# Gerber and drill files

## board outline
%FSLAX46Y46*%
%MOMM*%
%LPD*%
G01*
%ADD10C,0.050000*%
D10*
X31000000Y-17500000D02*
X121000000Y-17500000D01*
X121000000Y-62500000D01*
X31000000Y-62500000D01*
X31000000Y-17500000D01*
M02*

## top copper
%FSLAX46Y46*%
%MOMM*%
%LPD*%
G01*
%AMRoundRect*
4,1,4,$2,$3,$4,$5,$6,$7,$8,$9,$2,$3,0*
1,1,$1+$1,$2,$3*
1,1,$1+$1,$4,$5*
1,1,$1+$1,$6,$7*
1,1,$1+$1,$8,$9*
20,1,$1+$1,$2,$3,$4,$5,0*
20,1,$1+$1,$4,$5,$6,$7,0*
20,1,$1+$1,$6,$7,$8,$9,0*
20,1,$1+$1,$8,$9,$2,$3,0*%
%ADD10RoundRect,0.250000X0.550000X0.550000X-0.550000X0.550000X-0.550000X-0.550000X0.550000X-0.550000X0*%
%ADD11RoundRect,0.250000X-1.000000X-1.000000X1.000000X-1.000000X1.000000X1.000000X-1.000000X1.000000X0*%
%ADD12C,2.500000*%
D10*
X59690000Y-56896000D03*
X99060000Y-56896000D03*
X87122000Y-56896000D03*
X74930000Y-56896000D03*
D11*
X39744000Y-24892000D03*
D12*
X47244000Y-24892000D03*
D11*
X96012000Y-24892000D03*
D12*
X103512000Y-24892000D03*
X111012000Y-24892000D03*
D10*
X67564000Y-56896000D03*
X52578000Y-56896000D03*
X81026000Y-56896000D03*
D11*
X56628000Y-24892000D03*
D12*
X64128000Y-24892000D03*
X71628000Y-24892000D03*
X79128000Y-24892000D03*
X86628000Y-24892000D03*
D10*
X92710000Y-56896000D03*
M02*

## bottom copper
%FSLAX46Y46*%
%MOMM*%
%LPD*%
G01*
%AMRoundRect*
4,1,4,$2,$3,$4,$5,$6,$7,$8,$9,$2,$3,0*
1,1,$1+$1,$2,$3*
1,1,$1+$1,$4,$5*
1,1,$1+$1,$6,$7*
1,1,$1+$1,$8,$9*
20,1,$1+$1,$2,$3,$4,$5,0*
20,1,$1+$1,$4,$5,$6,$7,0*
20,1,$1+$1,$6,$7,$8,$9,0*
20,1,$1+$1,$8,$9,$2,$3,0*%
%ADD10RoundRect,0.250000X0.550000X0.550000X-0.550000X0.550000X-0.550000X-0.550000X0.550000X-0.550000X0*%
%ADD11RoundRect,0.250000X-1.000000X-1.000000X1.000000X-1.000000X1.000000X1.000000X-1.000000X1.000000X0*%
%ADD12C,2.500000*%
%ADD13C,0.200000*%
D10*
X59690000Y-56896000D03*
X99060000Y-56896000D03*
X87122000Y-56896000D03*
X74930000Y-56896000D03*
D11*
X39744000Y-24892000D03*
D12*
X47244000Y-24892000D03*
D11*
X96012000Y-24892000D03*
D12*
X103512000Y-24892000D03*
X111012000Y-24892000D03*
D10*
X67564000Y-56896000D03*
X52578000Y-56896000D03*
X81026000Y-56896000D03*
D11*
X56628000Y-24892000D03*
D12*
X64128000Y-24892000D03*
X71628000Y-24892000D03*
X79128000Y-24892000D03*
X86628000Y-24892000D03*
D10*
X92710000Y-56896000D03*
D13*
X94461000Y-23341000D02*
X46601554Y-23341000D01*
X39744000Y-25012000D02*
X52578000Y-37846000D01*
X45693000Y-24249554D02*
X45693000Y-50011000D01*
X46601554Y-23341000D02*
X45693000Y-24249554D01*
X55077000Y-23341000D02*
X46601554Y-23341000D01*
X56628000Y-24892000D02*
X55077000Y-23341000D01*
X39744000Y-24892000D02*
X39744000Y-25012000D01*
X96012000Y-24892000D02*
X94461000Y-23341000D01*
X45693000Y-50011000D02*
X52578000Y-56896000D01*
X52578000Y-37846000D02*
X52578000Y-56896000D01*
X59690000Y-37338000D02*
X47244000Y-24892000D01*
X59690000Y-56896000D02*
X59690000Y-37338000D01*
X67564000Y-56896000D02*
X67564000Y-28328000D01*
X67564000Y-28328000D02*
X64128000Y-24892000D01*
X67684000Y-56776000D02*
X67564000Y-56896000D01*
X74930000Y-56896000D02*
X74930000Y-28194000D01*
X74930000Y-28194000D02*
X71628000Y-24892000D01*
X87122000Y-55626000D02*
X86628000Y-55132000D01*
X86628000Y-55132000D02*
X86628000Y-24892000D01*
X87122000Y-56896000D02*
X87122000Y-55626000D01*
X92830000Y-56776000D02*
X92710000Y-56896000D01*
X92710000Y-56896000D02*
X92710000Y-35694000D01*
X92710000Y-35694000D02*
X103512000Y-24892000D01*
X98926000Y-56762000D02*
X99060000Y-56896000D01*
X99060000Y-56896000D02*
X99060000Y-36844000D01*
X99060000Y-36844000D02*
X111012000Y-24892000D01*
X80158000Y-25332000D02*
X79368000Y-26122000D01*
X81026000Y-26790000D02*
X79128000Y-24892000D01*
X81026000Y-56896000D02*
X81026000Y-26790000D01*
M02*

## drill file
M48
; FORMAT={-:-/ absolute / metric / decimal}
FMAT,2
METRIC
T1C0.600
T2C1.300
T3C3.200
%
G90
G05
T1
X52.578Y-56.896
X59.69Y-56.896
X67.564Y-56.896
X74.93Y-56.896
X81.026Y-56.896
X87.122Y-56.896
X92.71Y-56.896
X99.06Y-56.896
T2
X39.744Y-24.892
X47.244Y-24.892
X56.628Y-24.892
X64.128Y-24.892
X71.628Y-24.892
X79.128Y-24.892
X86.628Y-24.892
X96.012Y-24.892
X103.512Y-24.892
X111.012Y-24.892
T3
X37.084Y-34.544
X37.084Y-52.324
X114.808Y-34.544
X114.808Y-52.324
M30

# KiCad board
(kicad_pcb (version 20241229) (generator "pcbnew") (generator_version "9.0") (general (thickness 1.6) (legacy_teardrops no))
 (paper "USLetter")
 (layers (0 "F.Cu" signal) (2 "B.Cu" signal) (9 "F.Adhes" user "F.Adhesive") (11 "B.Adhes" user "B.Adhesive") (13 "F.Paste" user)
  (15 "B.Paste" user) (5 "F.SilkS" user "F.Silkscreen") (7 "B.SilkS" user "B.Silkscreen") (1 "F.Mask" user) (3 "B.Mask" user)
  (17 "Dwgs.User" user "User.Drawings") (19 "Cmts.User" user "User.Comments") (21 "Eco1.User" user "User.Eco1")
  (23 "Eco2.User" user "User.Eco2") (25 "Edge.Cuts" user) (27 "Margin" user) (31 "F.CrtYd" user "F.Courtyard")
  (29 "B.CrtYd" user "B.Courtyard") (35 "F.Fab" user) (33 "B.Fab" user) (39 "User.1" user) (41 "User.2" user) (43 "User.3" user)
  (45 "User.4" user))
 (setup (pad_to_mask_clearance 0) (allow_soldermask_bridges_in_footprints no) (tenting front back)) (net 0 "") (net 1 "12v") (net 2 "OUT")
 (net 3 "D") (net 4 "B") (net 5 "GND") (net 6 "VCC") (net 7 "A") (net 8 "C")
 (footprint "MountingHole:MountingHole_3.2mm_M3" (layer "F.Cu") (at 114.808 52.324)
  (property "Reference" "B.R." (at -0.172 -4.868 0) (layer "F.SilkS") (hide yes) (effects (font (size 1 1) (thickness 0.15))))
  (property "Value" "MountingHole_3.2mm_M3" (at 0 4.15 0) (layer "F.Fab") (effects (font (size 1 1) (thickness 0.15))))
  (pad "" np_thru_hole circle (at 0 0) (size 3.2 3.2) (drill 3.2) (layers "*.Cu" "*.Mask")))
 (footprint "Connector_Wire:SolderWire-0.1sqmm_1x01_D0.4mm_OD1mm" (layer "F.Cu") (at 59.69 56.896 180)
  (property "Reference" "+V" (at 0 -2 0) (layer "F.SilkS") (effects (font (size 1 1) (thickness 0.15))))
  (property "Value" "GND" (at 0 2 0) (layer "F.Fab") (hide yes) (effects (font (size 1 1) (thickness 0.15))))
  (pad "1" thru_hole roundrect (at 0 0 180) (size 1.6 1.6) (drill 0.6) (layers "*.Cu" "*.Mask") (remove_unused_layers no)
   (roundrect_rratio 0.15625) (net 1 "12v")))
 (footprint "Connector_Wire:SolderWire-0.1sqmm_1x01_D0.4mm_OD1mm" (layer "F.Cu") (at 99.06 56.896 180)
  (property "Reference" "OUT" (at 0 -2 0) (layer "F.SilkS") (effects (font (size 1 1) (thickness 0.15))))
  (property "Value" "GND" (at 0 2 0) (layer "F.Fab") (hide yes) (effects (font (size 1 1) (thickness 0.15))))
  (pad "1" thru_hole roundrect (at 0 0 180) (size 1.6 1.6) (drill 0.6) (layers "*.Cu" "*.Mask") (remove_unused_layers no)
   (roundrect_rratio 0.15625) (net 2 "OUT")))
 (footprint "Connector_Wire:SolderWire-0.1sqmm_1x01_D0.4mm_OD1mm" (layer "F.Cu") (at 87.122 56.896 180)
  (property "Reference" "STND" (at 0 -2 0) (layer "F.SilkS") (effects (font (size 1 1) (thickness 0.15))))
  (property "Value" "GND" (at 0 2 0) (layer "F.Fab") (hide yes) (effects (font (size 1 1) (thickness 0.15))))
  (pad "1" thru_hole roundrect (at 0 0 180) (size 1.6 1.6) (drill 0.6) (layers "*.Cu" "*.Mask") (remove_unused_layers no)
   (roundrect_rratio 0.15625) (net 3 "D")))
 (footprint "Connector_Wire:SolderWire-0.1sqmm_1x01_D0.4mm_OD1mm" (layer "F.Cu") (at 74.93 56.896 180)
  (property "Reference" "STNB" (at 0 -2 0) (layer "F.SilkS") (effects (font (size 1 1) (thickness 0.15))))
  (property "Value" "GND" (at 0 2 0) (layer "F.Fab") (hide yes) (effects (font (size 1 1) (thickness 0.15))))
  (pad "1" thru_hole roundrect (at 0 0 180) (size 1.6 1.6) (drill 0.6) (layers "*.Cu" "*.Mask") (remove_unused_layers no)
   (roundrect_rratio 0.15625) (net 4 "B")))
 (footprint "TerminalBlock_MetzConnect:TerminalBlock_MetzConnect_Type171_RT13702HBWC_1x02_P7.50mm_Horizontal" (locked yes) (layer "F.Cu")
  (at 39.744 24.892)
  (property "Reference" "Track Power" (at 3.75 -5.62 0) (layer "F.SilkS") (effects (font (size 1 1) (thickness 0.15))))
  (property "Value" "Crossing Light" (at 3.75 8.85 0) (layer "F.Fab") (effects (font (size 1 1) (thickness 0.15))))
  (pad "1" thru_hole roundrect (at 0 0) (size 2.5 2.5) (drill 1.3) (layers "*.Cu" "*.Mask") (remove_unused_layers no) (roundrect_rratio 0.1)
   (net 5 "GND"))
  (pad "2" thru_hole circle (at 7.5 0) (size 2.5 2.5) (drill 1.3) (layers "*.Cu" "*.Mask") (remove_unused_layers no) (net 1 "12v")))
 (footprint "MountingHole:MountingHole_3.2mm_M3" (layer "F.Cu") (at 37.084 34.544)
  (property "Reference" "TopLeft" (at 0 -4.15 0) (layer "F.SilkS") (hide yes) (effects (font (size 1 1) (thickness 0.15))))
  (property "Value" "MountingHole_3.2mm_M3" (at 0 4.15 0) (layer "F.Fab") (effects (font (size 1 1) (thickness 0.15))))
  (pad "" np_thru_hole circle (at 0 0) (size 3.2 3.2) (drill 3.2) (layers "*.Cu" "*.Mask")))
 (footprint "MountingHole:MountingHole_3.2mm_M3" (layer "F.Cu") (at 37.084 52.324)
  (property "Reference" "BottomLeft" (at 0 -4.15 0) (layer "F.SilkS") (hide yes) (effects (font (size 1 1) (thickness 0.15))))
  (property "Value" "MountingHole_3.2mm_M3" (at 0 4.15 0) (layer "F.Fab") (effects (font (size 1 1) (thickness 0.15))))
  (pad "" np_thru_hole circle (at 0 0) (size 3.2 3.2) (drill 3.2) (layers "*.Cu" "*.Mask")))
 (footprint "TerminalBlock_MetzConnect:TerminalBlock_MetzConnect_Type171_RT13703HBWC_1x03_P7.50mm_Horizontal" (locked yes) (layer "F.Cu")
  (at 96.012 24.892)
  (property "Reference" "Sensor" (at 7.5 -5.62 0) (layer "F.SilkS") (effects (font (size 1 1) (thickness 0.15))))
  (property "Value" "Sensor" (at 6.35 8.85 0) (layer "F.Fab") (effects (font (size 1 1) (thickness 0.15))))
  (pad "1" thru_hole roundrect (at 0 0) (size 2.5 2.5) (drill 1.3) (layers "*.Cu" "*.Mask") (remove_unused_layers no) (roundrect_rratio 0.1)
   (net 5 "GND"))
  (pad "2" thru_hole circle (at 7.5 0) (size 2.5 2.5) (drill 1.3) (layers "*.Cu" "*.Mask") (remove_unused_layers no) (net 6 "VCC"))
  (pad "3" thru_hole circle (at 15 0) (size 2.5 2.5) (drill 1.3) (layers "*.Cu" "*.Mask") (remove_unused_layers no) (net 2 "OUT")))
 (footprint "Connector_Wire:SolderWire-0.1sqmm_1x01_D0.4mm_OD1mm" (layer "F.Cu") (at 67.564 56.896 180)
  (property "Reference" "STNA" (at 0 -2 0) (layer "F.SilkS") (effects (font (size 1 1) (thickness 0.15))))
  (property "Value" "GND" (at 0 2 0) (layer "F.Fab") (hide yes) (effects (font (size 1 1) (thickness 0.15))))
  (pad "1" thru_hole roundrect (at 0 0 180) (size 1.6 1.6) (drill 0.6) (layers "*.Cu" "*.Mask") (remove_unused_layers no)
   (roundrect_rratio 0.15625) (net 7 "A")))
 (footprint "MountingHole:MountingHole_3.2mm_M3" (layer "F.Cu") (at 114.808 34.544)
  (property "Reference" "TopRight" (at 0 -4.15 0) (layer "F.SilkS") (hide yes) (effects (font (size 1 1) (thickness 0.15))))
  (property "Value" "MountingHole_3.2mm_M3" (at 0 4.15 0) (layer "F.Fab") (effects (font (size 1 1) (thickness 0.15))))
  (pad "" np_thru_hole circle (at 0 0) (size 3.2 3.2) (drill 3.2) (layers "*.Cu" "*.Mask")))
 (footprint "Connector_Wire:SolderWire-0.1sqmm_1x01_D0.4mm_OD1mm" (layer "F.Cu") (at 52.578 56.896 180)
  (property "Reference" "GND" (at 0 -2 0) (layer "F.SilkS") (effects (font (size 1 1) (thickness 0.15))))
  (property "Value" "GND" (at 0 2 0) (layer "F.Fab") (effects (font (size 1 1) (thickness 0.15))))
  (pad "1" thru_hole roundrect (at 0 0 180) (size 1.6 1.6) (drill 0.6) (layers "*.Cu" "*.Mask") (remove_unused_layers no)
   (roundrect_rratio 0.15625) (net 5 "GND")))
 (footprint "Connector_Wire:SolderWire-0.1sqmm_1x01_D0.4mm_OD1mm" (layer "F.Cu") (at 81.026 56.896 180)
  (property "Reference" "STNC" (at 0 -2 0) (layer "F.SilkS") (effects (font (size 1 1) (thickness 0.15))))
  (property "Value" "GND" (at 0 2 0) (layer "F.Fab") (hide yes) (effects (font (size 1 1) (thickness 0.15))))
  (pad "1" thru_hole roundrect (at 0 0 180) (size 1.6 1.6) (drill 0.6) (layers "*.Cu" "*.Mask") (remove_unused_layers no)
   (roundrect_rratio 0.15625) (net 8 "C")))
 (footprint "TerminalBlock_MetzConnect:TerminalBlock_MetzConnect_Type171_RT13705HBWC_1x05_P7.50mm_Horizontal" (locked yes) (layer "F.Cu")
  (at 56.628 24.892)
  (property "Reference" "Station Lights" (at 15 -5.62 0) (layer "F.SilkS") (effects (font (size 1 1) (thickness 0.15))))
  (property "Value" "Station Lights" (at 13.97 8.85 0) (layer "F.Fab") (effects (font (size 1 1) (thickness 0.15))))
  (pad "1" thru_hole roundrect (at 0 0) (size 2.5 2.5) (drill 1.3) (layers "*.Cu" "*.Mask") (remove_unused_layers no) (roundrect_rratio 0.1)
   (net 5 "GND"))
  (pad "2" thru_hole circle (at 7.5 0) (size 2.5 2.5) (drill 1.3) (layers "*.Cu" "*.Mask") (remove_unused_layers no) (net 7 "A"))
  (pad "3" thru_hole circle (at 15 0) (size 2.5 2.5) (drill 1.3) (layers "*.Cu" "*.Mask") (remove_unused_layers no) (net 4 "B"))
  (pad "4" thru_hole circle (at 22.5 0) (size 2.5 2.5) (drill 1.3) (layers "*.Cu" "*.Mask") (remove_unused_layers no) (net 8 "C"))
  (pad "5" thru_hole circle (at 30 0) (size 2.5 2.5) (drill 1.3) (layers "*.Cu" "*.Mask") (remove_unused_layers no) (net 3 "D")))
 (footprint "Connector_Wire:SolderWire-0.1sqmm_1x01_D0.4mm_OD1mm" (layer "F.Cu") (at 92.71 56.896 180)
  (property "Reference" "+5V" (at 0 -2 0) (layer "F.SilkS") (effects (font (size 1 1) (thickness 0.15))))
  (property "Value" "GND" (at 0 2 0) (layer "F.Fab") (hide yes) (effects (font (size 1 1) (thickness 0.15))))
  (pad "1" thru_hole roundrect (at 0 0 180) (size 1.6 1.6) (drill 0.6) (layers "*.Cu" "*.Mask") (remove_unused_layers no)
   (roundrect_rratio 0.15625) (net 6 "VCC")))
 (gr_rect (start 31 17.5) (end 121 62.5) (stroke (width 0.05) (type solid)) (fill no) (layer "Edge.Cuts"))
 (segment (start 94.461 23.341) (end 46.601554 23.341) (width 0.2) (layer "B.Cu") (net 5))
 (segment (start 39.744 25.012) (end 52.578 37.846) (width 0.2) (layer "B.Cu") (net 5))
 (segment (start 45.693 24.249554) (end 45.693 50.011) (width 0.2) (layer "B.Cu") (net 5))
 (segment (start 46.601554 23.341) (end 45.693 24.249554) (width 0.2) (layer "B.Cu") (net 5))
 (segment (start 55.077 23.341) (end 46.601554 23.341) (width 0.2) (layer "B.Cu") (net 5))
 (segment (start 56.628 24.892) (end 55.077 23.341) (width 0.2) (layer "B.Cu") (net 5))
 (segment (start 39.744 24.892) (end 39.744 25.012) (width 0.2) (layer "B.Cu") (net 5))
 (segment (start 96.012 24.892) (end 94.461 23.341) (width 0.2) (layer "B.Cu") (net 5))
 (segment (start 45.693 50.011) (end 52.578 56.896) (width 0.2) (layer "B.Cu") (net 5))
 (segment (start 52.578 37.846) (end 52.578 56.896) (width 0.2) (layer "B.Cu") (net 5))
 (segment (start 59.69 37.338) (end 47.244 24.892) (width 0.2) (layer "B.Cu") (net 1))
 (segment (start 59.69 56.896) (end 59.69 37.338) (width 0.2) (layer "B.Cu") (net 1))
 (segment (start 67.564 56.896) (end 67.564 28.328) (width 0.2) (layer "B.Cu") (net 7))
 (segment (start 67.564 28.328) (end 64.128 24.892) (width 0.2) (layer "B.Cu") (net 7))
 (segment (start 67.684 56.776) (end 67.564 56.896) (width 0.2) (layer "B.Cu") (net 7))
 (segment (start 74.93 56.896) (end 74.93 28.194) (width 0.2) (layer "B.Cu") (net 4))
 (segment (start 74.93 28.194) (end 71.628 24.892) (width 0.2) (layer "B.Cu") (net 4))
 (segment (start 87.122 55.626) (end 86.628 55.132) (width 0.2) (layer "B.Cu") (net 3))
 (segment (start 86.628 55.132) (end 86.628 24.892) (width 0.2) (layer "B.Cu") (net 3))
 (segment (start 87.122 56.896) (end 87.122 55.626) (width 0.2) (layer "B.Cu") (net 3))
 (segment (start 92.83 56.776) (end 92.71 56.896) (width 0.2) (layer "B.Cu") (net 6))
 (segment (start 92.71 56.896) (end 92.71 35.694) (width 0.2) (layer "B.Cu") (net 6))
 (segment (start 92.71 35.694) (end 103.512 24.892) (width 0.2) (layer "B.Cu") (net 6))
 (segment (start 98.926 56.762) (end 99.06 56.896) (width 0.2) (layer "B.Cu") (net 2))
 (segment (start 99.06 56.896) (end 99.06 36.844) (width 0.2) (layer "B.Cu") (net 2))
 (segment (start 99.06 36.844) (end 111.012 24.892) (width 0.2) (layer "B.Cu") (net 2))
 (segment (start 80.158 25.332) (end 79.368 26.122) (width 0.2) (layer "B.Cu") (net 8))
 (segment (start 81.026 26.79) (end 79.128 24.892) (width 0.2) (layer "B.Cu") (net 8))
 (segment (start 81.026 56.896) (end 81.026 26.79) (width 0.2) (layer "B.Cu") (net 8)))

